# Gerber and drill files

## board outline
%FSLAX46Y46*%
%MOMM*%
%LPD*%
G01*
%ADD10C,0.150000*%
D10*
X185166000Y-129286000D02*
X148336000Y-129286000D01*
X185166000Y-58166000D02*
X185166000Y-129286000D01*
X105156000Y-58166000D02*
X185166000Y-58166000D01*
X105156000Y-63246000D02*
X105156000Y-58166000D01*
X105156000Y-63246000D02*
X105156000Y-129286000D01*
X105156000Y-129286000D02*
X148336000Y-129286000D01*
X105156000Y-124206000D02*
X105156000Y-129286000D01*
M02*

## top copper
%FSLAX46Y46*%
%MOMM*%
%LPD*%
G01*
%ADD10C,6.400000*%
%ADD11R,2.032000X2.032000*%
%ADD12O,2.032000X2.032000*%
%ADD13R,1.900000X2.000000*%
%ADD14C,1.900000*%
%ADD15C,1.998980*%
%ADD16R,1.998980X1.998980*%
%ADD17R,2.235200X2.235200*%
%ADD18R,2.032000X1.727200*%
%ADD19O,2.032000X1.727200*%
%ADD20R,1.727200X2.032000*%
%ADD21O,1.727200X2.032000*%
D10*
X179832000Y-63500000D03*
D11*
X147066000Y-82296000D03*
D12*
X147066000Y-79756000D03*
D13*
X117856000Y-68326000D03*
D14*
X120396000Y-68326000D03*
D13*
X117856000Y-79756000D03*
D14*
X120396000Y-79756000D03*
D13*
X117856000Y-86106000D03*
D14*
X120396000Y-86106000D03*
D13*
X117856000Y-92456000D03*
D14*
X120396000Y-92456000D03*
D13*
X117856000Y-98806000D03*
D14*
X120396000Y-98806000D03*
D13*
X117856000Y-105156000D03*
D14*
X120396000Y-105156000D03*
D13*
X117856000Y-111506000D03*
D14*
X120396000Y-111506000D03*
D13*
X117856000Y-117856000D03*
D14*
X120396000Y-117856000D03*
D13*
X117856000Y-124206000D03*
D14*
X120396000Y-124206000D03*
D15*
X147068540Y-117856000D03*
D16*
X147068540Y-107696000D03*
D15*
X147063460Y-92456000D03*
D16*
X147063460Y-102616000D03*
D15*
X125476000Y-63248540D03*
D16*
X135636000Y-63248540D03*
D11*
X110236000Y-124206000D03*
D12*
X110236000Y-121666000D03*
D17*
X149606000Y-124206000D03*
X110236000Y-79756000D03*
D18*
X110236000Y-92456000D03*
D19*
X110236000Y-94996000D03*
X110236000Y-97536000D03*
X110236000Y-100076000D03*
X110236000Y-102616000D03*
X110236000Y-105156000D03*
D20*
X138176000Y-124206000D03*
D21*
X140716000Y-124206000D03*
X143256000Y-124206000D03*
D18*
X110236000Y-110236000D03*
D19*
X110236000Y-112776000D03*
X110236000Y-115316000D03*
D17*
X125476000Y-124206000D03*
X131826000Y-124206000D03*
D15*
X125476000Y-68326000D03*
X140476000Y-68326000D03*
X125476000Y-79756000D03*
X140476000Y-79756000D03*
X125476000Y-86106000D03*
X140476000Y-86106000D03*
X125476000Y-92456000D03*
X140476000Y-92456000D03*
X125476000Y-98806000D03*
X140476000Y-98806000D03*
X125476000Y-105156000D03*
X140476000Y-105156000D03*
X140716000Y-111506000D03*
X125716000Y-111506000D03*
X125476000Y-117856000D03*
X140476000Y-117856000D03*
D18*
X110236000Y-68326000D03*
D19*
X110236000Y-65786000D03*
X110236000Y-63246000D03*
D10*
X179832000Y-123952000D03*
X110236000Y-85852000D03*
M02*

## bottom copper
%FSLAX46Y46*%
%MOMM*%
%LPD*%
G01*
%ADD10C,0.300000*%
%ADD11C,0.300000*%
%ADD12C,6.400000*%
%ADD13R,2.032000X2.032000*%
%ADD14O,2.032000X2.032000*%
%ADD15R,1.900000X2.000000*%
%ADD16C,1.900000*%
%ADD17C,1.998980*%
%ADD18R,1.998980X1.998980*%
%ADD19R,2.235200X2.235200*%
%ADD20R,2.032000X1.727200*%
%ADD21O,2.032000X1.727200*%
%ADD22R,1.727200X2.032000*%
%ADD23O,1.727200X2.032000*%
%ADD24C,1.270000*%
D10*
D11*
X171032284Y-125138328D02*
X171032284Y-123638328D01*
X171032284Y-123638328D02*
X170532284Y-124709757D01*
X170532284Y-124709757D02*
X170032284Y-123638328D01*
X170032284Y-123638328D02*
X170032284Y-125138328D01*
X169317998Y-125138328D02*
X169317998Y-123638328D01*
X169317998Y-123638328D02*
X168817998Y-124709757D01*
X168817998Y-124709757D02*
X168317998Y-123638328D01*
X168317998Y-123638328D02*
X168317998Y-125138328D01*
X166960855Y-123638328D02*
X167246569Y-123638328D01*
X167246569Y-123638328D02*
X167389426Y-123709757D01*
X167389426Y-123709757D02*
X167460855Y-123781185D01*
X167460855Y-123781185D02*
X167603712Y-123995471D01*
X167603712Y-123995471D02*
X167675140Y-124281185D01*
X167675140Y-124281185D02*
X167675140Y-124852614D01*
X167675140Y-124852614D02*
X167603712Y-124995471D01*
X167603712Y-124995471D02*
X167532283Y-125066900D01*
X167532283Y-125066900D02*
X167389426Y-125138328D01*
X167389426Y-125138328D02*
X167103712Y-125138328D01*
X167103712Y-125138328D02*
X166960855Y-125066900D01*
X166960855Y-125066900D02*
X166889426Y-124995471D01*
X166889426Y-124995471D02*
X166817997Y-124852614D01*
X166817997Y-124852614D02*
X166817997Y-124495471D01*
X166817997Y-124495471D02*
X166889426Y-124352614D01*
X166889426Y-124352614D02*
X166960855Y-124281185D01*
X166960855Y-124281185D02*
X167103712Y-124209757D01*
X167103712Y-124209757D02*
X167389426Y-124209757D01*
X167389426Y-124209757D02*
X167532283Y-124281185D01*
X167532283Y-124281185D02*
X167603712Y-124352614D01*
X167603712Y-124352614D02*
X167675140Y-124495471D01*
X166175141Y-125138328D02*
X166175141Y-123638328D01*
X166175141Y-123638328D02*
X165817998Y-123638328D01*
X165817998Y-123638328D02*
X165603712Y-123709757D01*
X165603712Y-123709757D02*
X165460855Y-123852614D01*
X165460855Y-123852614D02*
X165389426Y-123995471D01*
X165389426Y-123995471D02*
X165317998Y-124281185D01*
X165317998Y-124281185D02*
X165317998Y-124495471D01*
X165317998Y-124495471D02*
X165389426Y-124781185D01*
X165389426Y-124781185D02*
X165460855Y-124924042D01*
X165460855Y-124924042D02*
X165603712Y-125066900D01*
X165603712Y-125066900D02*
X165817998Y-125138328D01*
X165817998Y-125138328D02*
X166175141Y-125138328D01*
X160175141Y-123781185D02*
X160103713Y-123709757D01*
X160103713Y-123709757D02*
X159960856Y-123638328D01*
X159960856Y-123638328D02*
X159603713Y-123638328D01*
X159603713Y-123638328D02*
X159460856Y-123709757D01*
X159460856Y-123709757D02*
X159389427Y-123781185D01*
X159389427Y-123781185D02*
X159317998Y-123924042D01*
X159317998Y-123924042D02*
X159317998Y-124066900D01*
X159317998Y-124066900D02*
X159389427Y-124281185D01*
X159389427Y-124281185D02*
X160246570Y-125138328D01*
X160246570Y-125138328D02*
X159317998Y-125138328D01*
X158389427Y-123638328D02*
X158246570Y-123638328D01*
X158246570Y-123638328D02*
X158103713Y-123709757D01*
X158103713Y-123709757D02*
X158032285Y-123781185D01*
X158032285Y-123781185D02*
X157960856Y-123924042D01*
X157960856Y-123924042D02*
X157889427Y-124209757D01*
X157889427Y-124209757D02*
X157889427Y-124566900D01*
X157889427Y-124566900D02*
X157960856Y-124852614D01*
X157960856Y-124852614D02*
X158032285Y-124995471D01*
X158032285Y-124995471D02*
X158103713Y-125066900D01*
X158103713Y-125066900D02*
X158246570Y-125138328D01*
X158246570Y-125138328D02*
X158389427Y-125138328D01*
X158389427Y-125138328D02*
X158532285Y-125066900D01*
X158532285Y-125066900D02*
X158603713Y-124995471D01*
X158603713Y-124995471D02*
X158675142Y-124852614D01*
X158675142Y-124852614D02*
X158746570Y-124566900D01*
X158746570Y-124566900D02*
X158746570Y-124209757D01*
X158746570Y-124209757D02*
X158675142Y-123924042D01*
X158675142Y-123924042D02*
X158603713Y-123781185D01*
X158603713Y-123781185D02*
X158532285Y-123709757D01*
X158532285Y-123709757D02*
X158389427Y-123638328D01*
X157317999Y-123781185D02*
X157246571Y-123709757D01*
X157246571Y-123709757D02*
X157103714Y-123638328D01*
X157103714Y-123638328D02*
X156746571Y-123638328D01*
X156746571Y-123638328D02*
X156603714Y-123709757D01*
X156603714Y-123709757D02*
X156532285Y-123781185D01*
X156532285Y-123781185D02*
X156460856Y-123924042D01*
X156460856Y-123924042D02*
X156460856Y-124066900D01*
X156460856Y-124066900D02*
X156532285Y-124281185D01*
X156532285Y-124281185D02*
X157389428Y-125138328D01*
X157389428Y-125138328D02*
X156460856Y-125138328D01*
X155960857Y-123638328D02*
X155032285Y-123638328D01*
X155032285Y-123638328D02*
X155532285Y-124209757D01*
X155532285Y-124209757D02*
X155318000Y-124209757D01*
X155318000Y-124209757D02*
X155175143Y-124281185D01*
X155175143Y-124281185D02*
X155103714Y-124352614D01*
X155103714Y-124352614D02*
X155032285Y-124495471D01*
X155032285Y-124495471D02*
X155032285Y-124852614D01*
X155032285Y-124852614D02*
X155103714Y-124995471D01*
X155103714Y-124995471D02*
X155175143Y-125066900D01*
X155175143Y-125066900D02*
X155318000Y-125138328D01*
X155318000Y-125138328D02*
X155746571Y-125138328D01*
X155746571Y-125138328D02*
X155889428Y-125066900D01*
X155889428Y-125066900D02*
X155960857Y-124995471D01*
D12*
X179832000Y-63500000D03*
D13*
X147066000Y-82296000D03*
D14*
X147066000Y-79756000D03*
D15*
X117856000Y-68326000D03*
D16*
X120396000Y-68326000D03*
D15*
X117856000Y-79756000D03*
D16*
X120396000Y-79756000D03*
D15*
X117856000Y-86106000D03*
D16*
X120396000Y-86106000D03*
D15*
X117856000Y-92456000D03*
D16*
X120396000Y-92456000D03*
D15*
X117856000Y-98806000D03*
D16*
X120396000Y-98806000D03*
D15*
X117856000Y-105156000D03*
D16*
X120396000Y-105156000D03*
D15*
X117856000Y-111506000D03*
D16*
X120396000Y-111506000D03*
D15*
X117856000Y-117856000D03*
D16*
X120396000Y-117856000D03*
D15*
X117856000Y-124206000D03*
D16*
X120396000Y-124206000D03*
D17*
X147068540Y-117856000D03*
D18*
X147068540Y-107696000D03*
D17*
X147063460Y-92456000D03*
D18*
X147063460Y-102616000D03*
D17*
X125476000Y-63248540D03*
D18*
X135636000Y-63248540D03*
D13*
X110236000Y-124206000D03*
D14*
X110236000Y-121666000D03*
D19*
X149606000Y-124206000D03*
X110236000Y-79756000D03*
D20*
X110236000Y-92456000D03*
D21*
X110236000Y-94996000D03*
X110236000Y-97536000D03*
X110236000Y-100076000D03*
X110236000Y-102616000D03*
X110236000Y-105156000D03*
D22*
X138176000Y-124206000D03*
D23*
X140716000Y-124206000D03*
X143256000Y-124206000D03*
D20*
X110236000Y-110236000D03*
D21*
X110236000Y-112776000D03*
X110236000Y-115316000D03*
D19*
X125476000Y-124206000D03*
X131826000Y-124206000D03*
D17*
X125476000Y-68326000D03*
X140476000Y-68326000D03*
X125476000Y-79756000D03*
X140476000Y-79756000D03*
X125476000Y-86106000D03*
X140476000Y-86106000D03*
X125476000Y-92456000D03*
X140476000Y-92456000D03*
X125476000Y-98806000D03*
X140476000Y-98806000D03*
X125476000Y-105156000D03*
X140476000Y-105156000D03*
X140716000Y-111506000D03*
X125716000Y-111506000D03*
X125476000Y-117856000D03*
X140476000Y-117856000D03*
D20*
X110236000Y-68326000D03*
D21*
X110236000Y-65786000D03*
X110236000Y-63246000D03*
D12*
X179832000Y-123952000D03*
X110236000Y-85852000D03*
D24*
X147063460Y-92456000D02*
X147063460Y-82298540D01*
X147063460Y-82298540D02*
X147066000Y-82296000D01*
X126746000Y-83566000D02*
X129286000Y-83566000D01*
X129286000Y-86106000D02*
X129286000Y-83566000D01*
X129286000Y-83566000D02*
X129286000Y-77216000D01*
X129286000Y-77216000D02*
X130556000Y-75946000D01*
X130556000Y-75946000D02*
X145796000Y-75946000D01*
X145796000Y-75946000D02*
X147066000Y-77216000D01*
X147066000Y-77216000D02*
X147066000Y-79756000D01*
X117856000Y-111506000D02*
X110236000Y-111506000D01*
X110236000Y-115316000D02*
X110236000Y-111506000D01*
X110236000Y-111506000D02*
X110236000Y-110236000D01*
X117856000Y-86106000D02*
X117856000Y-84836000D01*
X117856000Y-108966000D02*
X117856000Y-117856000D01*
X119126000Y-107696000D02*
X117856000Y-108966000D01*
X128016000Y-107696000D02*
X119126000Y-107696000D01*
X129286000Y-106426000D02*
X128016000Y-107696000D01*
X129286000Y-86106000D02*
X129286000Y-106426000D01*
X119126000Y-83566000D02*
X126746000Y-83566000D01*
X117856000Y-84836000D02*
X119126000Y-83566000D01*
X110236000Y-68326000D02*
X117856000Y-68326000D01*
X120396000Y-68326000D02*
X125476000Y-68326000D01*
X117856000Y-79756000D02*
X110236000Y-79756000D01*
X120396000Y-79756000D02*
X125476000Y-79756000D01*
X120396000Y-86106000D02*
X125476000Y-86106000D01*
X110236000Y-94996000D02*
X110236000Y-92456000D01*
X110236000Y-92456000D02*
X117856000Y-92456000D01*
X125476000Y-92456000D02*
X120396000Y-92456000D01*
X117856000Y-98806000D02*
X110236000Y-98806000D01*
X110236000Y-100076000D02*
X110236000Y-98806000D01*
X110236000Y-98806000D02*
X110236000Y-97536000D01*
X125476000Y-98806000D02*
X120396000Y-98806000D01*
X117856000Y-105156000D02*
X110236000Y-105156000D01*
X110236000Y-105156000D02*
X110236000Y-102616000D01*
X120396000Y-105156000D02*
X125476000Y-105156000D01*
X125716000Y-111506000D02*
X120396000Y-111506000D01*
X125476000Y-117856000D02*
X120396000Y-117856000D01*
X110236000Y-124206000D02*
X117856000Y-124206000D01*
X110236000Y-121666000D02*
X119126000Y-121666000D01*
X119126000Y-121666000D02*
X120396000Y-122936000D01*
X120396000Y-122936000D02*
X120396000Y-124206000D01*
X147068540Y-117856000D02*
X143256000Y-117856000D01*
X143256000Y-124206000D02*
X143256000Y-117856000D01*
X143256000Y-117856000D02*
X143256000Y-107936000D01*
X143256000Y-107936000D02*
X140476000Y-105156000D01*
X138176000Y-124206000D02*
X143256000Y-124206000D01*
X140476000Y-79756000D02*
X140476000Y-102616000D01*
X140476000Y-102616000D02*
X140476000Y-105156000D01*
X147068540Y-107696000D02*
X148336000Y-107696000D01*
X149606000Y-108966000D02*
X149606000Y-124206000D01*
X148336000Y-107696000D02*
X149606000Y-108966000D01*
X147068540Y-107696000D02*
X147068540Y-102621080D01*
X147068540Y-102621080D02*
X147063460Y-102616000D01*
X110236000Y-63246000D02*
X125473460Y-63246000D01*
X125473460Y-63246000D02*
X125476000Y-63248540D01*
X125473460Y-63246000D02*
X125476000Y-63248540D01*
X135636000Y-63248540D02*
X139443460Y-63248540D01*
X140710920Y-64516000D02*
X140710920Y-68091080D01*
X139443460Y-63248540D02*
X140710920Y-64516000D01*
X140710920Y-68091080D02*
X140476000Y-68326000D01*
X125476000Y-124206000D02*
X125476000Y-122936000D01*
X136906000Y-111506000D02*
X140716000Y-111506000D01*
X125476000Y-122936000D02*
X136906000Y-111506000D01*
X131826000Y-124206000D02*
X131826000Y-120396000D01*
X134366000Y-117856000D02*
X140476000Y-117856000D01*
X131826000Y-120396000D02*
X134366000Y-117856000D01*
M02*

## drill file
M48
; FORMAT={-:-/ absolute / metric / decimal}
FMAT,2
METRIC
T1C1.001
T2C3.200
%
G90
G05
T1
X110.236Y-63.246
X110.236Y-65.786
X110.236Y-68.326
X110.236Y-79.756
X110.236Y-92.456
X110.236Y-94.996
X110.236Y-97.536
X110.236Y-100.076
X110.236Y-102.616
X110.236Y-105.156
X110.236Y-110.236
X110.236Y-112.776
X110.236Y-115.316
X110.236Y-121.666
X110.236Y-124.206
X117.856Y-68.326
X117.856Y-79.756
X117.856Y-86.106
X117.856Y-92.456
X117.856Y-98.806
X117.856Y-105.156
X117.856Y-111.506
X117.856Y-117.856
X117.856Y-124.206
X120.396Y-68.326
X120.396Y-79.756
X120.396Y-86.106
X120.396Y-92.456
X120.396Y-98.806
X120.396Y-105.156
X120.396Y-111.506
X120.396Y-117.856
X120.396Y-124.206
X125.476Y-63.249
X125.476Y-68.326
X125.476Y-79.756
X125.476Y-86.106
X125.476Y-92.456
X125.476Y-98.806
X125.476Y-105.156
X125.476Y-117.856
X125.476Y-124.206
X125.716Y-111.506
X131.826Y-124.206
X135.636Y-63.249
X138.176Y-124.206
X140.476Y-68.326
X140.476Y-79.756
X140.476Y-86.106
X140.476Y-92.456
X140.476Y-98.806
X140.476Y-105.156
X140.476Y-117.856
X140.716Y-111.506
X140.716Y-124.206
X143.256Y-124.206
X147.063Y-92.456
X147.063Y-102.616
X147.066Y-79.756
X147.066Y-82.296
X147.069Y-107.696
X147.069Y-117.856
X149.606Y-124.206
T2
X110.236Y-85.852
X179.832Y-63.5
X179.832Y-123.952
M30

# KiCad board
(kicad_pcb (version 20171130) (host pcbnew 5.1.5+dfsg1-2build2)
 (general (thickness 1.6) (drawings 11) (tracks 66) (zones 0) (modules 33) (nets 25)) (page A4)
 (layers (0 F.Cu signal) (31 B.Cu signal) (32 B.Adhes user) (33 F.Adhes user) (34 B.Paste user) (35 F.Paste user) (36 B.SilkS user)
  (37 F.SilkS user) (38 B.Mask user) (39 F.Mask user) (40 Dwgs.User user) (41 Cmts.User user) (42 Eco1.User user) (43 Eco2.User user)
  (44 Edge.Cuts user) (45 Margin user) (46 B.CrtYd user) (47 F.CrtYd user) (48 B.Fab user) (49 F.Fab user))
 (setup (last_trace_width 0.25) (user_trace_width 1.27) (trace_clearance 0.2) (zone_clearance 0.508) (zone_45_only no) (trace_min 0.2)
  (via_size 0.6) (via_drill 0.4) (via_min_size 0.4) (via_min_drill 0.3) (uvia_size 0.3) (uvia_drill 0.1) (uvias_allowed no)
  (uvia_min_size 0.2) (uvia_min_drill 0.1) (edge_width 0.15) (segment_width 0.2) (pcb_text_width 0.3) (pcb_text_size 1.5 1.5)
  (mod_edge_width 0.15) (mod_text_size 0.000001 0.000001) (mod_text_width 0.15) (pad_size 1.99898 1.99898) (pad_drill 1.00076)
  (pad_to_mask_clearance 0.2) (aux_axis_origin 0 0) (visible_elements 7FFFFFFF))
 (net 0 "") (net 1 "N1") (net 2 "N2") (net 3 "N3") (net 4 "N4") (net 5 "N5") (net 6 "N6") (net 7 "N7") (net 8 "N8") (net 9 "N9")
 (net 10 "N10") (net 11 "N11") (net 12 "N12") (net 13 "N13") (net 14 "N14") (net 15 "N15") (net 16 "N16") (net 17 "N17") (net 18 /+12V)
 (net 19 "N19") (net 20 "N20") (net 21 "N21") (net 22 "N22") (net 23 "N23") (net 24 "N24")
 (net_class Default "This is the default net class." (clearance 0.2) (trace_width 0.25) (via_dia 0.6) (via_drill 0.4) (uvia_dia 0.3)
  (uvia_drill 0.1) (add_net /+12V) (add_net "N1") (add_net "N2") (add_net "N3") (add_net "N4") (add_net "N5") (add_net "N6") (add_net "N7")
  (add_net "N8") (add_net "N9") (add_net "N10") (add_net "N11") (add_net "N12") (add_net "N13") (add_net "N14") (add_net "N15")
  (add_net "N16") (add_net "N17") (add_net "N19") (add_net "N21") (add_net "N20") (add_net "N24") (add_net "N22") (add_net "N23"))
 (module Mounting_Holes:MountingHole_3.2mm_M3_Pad (layer F.Cu) (at 179.832 63.5)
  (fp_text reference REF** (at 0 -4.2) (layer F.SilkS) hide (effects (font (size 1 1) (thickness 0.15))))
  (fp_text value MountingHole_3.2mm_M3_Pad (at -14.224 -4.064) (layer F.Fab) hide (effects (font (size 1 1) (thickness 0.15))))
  (pad 1 thru_hole circle (at 0 0) (size 6.4 6.4) (drill 3.2) (layers *.Cu *.Mask)))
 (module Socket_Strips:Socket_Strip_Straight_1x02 (layer F.Cu) (at 147.066 82.296 90)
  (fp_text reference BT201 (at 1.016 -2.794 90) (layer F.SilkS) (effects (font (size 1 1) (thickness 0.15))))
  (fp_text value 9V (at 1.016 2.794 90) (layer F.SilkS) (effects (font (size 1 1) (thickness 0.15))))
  (pad 1 thru_hole rect (at 0 0 90) (size 2.032 2.032) (drill 1.00076) (layers *.Cu *.Mask) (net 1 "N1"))
  (pad 2 thru_hole oval (at 2.54 0 90) (size 2.032 2.032) (drill 1.00076) (layers *.Cu *.Mask) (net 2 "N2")))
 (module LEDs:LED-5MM (layer F.Cu) (at 117.856 68.326)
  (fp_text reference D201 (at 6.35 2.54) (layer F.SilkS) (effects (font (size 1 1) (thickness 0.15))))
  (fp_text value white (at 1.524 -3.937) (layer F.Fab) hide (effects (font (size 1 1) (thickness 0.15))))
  (pad 1 thru_hole rect (at 0 0 90) (size 2 1.9) (drill 1.00076) (layers *.Cu *.Mask) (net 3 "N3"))
  (pad 2 thru_hole circle (at 2.54 0) (size 1.9 1.9) (drill 1.00076) (layers *.Cu *.Mask) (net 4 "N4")))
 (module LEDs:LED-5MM (layer F.Cu) (at 117.856 79.756)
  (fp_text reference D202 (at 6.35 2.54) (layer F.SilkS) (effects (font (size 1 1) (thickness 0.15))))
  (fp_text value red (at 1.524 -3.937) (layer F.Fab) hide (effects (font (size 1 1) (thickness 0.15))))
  (pad 1 thru_hole rect (at 0 0 90) (size 2 1.9) (drill 1.00076) (layers *.Cu *.Mask) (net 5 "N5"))
  (pad 2 thru_hole circle (at 2.54 0) (size 1.9 1.9) (drill 1.00076) (layers *.Cu *.Mask) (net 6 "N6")))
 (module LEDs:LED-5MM (layer F.Cu) (at 117.856 86.106)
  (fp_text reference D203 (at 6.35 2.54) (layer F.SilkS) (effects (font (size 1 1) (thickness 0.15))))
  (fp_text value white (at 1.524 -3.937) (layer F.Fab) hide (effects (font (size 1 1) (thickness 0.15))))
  (pad 1 thru_hole rect (at 0 0 90) (size 2 1.9) (drill 1.00076) (layers *.Cu *.Mask) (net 2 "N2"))
  (pad 2 thru_hole circle (at 2.54 0) (size 1.9 1.9) (drill 1.00076) (layers *.Cu *.Mask) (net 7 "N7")))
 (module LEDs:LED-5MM (layer F.Cu) (at 117.856 92.456)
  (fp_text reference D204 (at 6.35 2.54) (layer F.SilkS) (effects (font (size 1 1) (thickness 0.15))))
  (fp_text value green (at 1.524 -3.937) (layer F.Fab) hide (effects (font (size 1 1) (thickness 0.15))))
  (pad 1 thru_hole rect (at 0 0 90) (size 2 1.9) (drill 1.00076) (layers *.Cu *.Mask) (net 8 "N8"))
  (pad 2 thru_hole circle (at 2.54 0) (size 1.9 1.9) (drill 1.00076) (layers *.Cu *.Mask) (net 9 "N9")))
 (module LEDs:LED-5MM (layer F.Cu) (at 117.856 98.806)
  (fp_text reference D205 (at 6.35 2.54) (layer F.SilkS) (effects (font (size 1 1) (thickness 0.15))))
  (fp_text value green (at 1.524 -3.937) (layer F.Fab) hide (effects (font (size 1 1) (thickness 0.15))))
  (pad 1 thru_hole rect (at 0 0 90) (size 2 1.9) (drill 1.00076) (layers *.Cu *.Mask) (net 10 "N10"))
  (pad 2 thru_hole circle (at 2.54 0) (size 1.9 1.9) (drill 1.00076) (layers *.Cu *.Mask) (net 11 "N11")))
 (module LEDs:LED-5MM (layer F.Cu) (at 117.856 105.156)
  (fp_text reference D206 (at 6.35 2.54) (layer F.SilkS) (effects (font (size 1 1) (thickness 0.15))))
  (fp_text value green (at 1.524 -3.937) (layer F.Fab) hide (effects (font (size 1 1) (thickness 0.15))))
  (pad 1 thru_hole rect (at 0 0 90) (size 2 1.9) (drill 1.00076) (layers *.Cu *.Mask) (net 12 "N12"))
  (pad 2 thru_hole circle (at 2.54 0) (size 1.9 1.9) (drill 1.00076) (layers *.Cu *.Mask) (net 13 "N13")))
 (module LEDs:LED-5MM (layer F.Cu) (at 117.856 111.506)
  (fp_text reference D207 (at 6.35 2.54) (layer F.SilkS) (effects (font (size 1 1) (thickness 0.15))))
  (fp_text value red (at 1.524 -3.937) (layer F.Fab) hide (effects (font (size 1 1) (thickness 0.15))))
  (pad 1 thru_hole rect (at 0 0 90) (size 2 1.9) (drill 1.00076) (layers *.Cu *.Mask) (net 2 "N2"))
  (pad 2 thru_hole circle (at 2.54 0) (size 1.9 1.9) (drill 1.00076) (layers *.Cu *.Mask) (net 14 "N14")))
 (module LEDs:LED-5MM (layer F.Cu) (at 117.856 117.856)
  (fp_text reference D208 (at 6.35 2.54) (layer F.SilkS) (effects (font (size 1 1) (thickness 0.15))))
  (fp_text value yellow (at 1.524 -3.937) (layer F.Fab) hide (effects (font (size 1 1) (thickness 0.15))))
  (pad 1 thru_hole rect (at 0 0 90) (size 2 1.9) (drill 1.00076) (layers *.Cu *.Mask) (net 2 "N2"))
  (pad 2 thru_hole circle (at 2.54 0) (size 1.9 1.9) (drill 1.00076) (layers *.Cu *.Mask) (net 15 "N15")))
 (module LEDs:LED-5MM (layer F.Cu) (at 117.856 124.206)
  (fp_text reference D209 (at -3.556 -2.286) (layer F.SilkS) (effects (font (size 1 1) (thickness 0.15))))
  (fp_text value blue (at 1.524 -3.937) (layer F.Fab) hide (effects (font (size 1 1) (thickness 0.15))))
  (pad 1 thru_hole rect (at 0 0 90) (size 2 1.9) (drill 1.00076) (layers *.Cu *.Mask) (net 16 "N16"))
  (pad 2 thru_hole circle (at 2.54 0) (size 1.9 1.9) (drill 1.00076) (layers *.Cu *.Mask) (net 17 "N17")))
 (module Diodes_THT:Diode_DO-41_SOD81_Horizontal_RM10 (layer F.Cu) (at 147.066 107.696 270)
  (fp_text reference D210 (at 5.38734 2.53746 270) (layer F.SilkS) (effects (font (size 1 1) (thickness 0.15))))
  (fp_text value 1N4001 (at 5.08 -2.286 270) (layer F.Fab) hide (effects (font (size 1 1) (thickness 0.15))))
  (pad 2 thru_hole circle (at 10.16 -0.00254 90) (size 1.99898 1.99898) (drill 1.00076) (layers *.Cu *.Mask) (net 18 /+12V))
  (pad 1 thru_hole rect (at 0 -0.00254 90) (size 1.99898 1.99898) (drill 1.00076) (layers *.Cu *.Mask) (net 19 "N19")))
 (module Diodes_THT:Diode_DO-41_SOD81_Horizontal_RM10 (layer F.Cu) (at 147.066 102.616 90)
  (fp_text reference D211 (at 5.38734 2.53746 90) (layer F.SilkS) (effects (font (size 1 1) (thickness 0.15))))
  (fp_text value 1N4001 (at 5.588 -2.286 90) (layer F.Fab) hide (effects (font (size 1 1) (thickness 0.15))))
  (pad 2 thru_hole circle (at 10.16 -0.00254 270) (size 1.99898 1.99898) (drill 1.00076) (layers *.Cu *.Mask) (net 1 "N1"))
  (pad 1 thru_hole rect (at 0 -0.00254 270) (size 1.99898 1.99898) (drill 1.00076) (layers *.Cu *.Mask) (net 19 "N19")))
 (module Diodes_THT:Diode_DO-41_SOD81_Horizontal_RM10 (layer F.Cu) (at 135.636 63.246 180)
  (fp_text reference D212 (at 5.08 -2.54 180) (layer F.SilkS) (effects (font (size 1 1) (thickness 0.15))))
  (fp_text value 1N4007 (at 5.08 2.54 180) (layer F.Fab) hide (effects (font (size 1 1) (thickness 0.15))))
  (pad 2 thru_hole circle (at 10.16 -0.00254) (size 1.99898 1.99898) (drill 1.00076) (layers *.Cu *.Mask) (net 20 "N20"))
  (pad 1 thru_hole rect (at 0 -0.00254) (size 1.99898 1.99898) (drill 1.00076) (layers *.Cu *.Mask) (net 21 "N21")))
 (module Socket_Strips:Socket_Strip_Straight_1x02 (layer F.Cu) (at 110.236 124.206 90)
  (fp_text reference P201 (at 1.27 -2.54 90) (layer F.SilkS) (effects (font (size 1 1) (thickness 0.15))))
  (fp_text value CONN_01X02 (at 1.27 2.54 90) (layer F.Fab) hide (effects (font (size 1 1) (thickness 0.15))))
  (pad 1 thru_hole rect (at 0 0 90) (size 2.032 2.032) (drill 1.00076) (layers *.Cu *.Mask) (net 16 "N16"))
  (pad 2 thru_hole oval (at 2.54 0 90) (size 2.032 2.032) (drill 1.00076) (layers *.Cu *.Mask) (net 17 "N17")))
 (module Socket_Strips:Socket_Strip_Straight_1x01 (layer F.Cu) (at 149.606 124.206)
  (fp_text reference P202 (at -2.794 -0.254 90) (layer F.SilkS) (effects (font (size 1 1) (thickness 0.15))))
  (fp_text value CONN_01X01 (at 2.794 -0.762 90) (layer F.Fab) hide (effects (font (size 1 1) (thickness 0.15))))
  (pad 1 thru_hole rect (at 0 0) (size 2.2352 2.2352) (drill 1.00076) (layers *.Cu *.Mask) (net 19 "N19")))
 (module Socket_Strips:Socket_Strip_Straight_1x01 (layer F.Cu) (at 110.236 79.756 270)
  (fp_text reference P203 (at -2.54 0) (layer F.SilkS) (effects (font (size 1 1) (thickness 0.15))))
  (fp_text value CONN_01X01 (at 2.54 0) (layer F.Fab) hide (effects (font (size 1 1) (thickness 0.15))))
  (pad 1 thru_hole rect (at 0 0 270) (size 2.2352 2.2352) (drill 1.00076) (layers *.Cu *.Mask) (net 5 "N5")))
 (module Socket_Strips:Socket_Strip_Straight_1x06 (layer F.Cu) (at 110.236 92.456 270)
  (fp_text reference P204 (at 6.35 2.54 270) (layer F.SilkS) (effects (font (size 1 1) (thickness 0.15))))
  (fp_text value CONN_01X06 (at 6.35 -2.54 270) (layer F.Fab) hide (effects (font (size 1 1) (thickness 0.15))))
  (pad 1 thru_hole rect (at 0 0 270) (size 1.7272 2.032) (drill 1.00076) (layers *.Cu *.Mask) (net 8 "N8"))
  (pad 2 thru_hole oval (at 2.54 0 270) (size 1.7272 2.032) (drill 1.00076) (layers *.Cu *.Mask) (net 8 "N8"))
  (pad 3 thru_hole oval (at 5.08 0 270) (size 1.7272 2.032) (drill 1.00076) (layers *.Cu *.Mask) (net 10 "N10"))
  (pad 4 thru_hole oval (at 7.62 0 270) (size 1.7272 2.032) (drill 1.00076) (layers *.Cu *.Mask) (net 10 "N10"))
  (pad 5 thru_hole oval (at 10.16 0 270) (size 1.7272 2.032) (drill 1.00076) (layers *.Cu *.Mask) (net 12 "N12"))
  (pad 6 thru_hole oval (at 12.7 0 270) (size 1.7272 2.032) (drill 1.00076) (layers *.Cu *.Mask) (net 12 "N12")))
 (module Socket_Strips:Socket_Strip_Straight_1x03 (layer F.Cu) (at 138.176 124.206)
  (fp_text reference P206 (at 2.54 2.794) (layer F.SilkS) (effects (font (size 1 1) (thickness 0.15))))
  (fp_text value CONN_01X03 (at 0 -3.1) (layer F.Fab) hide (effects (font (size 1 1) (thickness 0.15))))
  (pad 1 thru_hole rect (at 0 0) (size 1.7272 2.032) (drill 1.00076) (layers *.Cu *.Mask) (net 18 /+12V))
  (pad 2 thru_hole oval (at 2.54 0) (size 1.7272 2.032) (drill 1.00076) (layers *.Cu *.Mask) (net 18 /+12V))
  (pad 3 thru_hole oval (at 5.08 0) (size 1.7272 2.032) (drill 1.00076) (layers *.Cu *.Mask) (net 18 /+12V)))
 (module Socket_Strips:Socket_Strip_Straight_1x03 (layer F.Cu) (at 110.236 110.236 270)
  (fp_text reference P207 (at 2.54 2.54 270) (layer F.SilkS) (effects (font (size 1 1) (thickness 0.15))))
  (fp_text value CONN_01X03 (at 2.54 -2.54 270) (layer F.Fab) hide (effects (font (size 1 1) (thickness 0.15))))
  (pad 1 thru_hole rect (at 0 0 270) (size 1.7272 2.032) (drill 1.00076) (layers *.Cu *.Mask) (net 2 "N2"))
  (pad 2 thru_hole oval (at 2.54 0 270) (size 1.7272 2.032) (drill 1.00076) (layers *.Cu *.Mask) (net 2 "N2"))
  (pad 3 thru_hole oval (at 5.08 0 270) (size 1.7272 2.032) (drill 1.00076) (layers *.Cu *.Mask) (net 2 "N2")))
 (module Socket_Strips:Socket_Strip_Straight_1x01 (layer F.Cu) (at 125.476 124.206)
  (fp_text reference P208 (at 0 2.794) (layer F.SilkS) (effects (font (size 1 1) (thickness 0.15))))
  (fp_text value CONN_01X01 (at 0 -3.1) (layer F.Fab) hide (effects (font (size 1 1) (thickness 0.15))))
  (pad 1 thru_hole rect (at 0 0) (size 2.2352 2.2352) (drill 1.00076) (layers *.Cu *.Mask) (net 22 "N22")))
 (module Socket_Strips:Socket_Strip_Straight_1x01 (layer F.Cu) (at 131.826 124.206)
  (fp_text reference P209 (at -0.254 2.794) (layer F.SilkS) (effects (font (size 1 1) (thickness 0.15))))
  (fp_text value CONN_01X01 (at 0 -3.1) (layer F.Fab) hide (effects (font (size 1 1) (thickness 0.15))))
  (pad 1 thru_hole rect (at 0 0) (size 2.2352 2.2352) (drill 1.00076) (layers *.Cu *.Mask) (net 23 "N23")))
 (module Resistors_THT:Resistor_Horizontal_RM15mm (layer F.Cu) (at 125.476 68.326)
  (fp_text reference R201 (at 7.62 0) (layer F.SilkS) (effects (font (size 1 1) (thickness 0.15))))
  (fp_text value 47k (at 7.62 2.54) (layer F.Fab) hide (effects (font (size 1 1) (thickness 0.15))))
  (pad 1 thru_hole circle (at 0 0) (size 1.99898 1.99898) (drill 1.00076) (layers *.Cu *.SilkS *.Mask) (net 4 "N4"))
  (pad 2 thru_hole circle (at 15 0) (size 1.99898 1.99898) (drill 1.00076) (layers *.Cu *.SilkS *.Mask) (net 21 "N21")))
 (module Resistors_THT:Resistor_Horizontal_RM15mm (layer F.Cu) (at 125.476 79.756)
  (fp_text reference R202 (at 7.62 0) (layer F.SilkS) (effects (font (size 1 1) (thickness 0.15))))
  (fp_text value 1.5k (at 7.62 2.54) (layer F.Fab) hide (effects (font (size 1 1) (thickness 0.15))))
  (pad 1 thru_hole circle (at 0 0) (size 1.99898 1.99898) (drill 1.00076) (layers *.Cu *.SilkS *.Mask) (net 6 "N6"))
  (pad 2 thru_hole circle (at 15 0) (size 1.99898 1.99898) (drill 1.00076) (layers *.Cu *.SilkS *.Mask) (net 18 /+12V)))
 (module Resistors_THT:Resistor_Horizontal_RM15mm (layer F.Cu) (at 125.476 86.106)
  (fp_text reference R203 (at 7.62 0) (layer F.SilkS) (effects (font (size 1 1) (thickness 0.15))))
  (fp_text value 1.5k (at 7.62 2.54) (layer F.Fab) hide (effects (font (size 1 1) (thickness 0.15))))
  (pad 1 thru_hole circle (at 0 0) (size 1.99898 1.99898) (drill 1.00076) (layers *.Cu *.SilkS *.Mask) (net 7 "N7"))
  (pad 2 thru_hole circle (at 15 0) (size 1.99898 1.99898) (drill 1.00076) (layers *.Cu *.SilkS *.Mask) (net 18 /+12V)))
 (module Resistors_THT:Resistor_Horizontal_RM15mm (layer F.Cu) (at 125.476 92.456)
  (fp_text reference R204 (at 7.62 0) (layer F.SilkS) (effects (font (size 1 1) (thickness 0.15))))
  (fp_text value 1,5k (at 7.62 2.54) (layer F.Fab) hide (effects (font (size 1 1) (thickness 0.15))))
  (pad 1 thru_hole circle (at 0 0) (size 1.99898 1.99898) (drill 1.00076) (layers *.Cu *.SilkS *.Mask) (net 9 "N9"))
  (pad 2 thru_hole circle (at 15 0) (size 1.99898 1.99898) (drill 1.00076) (layers *.Cu *.SilkS *.Mask) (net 18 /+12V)))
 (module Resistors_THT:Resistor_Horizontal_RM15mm (layer F.Cu) (at 125.476 98.806)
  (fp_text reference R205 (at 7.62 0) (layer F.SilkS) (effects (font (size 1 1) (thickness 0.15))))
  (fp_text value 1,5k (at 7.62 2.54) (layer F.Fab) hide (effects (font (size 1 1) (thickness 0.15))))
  (pad 1 thru_hole circle (at 0 0) (size 1.99898 1.99898) (drill 1.00076) (layers *.Cu *.SilkS *.Mask) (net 11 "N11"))
  (pad 2 thru_hole circle (at 15 0) (size 1.99898 1.99898) (drill 1.00076) (layers *.Cu *.SilkS *.Mask) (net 18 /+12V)))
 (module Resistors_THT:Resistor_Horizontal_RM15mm (layer F.Cu) (at 125.476 105.156)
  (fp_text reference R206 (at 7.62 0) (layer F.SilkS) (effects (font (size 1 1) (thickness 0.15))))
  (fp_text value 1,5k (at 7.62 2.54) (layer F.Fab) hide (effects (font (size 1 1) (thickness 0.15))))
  (pad 1 thru_hole circle (at 0 0) (size 1.99898 1.99898) (drill 1.00076) (layers *.Cu *.SilkS *.Mask) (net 13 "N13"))
  (pad 2 thru_hole circle (at 15 0) (size 1.99898 1.99898) (drill 1.00076) (layers *.Cu *.SilkS *.Mask) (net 18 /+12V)))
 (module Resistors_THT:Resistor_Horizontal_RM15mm (layer F.Cu) (at 140.716 111.506 180)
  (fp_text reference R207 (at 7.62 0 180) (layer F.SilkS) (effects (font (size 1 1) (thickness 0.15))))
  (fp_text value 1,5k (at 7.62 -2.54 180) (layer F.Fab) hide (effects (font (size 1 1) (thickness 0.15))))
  (pad 1 thru_hole circle (at 0 0 180) (size 1.99898 1.99898) (drill 1.00076) (layers *.Cu *.SilkS *.Mask) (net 22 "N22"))
  (pad 2 thru_hole circle (at 15 0 180) (size 1.99898 1.99898) (drill 1.00076) (layers *.Cu *.SilkS *.Mask) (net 14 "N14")))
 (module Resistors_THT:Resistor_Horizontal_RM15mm (layer F.Cu) (at 125.476 117.856)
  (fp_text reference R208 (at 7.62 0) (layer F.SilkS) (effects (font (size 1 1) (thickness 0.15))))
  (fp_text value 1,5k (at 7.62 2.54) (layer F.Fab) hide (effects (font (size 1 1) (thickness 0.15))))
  (pad 1 thru_hole circle (at 0 0) (size 1.99898 1.99898) (drill 1.00076) (layers *.Cu *.SilkS *.Mask) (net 15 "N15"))
  (pad 2 thru_hole circle (at 15 0) (size 1.99898 1.99898) (drill 1.00076) (layers *.Cu *.SilkS *.Mask) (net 23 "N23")))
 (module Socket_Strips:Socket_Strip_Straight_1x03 (layer F.Cu) (at 110.236 68.326 90)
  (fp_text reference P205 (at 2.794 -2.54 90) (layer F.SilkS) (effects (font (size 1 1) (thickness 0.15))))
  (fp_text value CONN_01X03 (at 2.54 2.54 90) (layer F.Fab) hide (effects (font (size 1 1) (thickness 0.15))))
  (pad 1 thru_hole rect (at 0 0 90) (size 1.7272 2.032) (drill 1.00076) (layers *.Cu *.Mask) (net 3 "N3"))
  (pad 2 thru_hole oval (at 2.54 0 90) (size 1.7272 2.032) (drill 1.00076) (layers *.Cu *.Mask) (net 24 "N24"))
  (pad 3 thru_hole oval (at 5.08 0 90) (size 1.7272 2.032) (drill 1.00076) (layers *.Cu *.Mask) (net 20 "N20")))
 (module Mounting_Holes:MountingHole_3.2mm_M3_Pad (layer F.Cu) (at 179.832 123.952)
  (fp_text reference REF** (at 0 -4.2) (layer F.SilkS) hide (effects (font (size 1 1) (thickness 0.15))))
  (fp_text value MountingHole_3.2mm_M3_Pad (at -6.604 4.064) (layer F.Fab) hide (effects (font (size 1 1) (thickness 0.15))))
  (pad 1 thru_hole circle (at 0 0) (size 6.4 6.4) (drill 3.2) (layers *.Cu *.Mask)))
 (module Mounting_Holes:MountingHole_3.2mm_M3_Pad (layer F.Cu) (at 110.236 85.852)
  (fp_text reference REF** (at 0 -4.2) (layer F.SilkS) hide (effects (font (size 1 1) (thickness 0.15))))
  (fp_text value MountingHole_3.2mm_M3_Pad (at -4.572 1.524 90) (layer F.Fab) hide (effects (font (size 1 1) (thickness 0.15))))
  (pad 1 thru_hole circle (at 0 0) (size 6.4 6.4) (drill 3.2) (layers *.Cu *.Mask)))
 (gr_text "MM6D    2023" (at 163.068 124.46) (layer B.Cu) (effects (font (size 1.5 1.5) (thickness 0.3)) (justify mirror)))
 (gr_line (start 185.166 129.286) (end 148.336 129.286) (angle 90) (layer Edge.Cuts) (width 0.15))
 (gr_line (start 185.166 58.166) (end 185.166 129.286) (angle 90) (layer Edge.Cuts) (width 0.15))
 (gr_line (start 105.156 58.166) (end 185.166 58.166) (angle 90) (layer Edge.Cuts) (width 0.15))
 (gr_line (start 105.156 63.246) (end 105.156 58.166) (angle 90) (layer Edge.Cuts) (width 0.15))
 (gr_line (start 105.156 63.246) (end 105.156 129.286) (angle 90) (layer Edge.Cuts) (width 0.15))
 (gr_line (start 105.156 129.286) (end 148.336 129.286) (angle 90) (layer Edge.Cuts) (width 0.15))
 (gr_line (start 105.156 124.206) (end 105.156 129.286) (angle 90) (layer Edge.Cuts) (width 0.15))
 (segment (start 147.06346 92.456) (end 147.06346 82.29854) (width 1.27) (layer B.Cu) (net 1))
 (segment (start 147.06346 82.29854) (end 147.066 82.296) (width 1.27) (layer B.Cu) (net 1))
 (segment (start 126.746 83.566) (end 129.286 83.566) (width 1.27) (layer B.Cu) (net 2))
 (segment (start 129.286 86.106) (end 129.286 83.566) (width 1.27) (layer B.Cu) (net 2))
 (segment (start 129.286 83.566) (end 129.286 77.216) (width 1.27) (layer B.Cu) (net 2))
 (segment (start 129.286 77.216) (end 130.556 75.946) (width 1.27) (layer B.Cu) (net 2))
 (segment (start 130.556 75.946) (end 145.796 75.946) (width 1.27) (layer B.Cu) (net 2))
 (segment (start 145.796 75.946) (end 147.066 77.216) (width 1.27) (layer B.Cu) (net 2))
 (segment (start 147.066 77.216) (end 147.066 79.756) (width 1.27) (layer B.Cu) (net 2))
 (segment (start 117.856 111.506) (end 110.236 111.506) (width 1.27) (layer B.Cu) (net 2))
 (segment (start 110.236 115.316) (end 110.236 111.506) (width 1.27) (layer B.Cu) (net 2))
 (segment (start 110.236 111.506) (end 110.236 110.236) (width 1.27) (layer B.Cu) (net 2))
 (segment (start 117.856 86.106) (end 117.856 84.836) (width 1.27) (layer B.Cu) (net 2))
 (segment (start 117.856 108.966) (end 117.856 117.856) (width 1.27) (layer B.Cu) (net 2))
 (segment (start 119.126 107.696) (end 117.856 108.966) (width 1.27) (layer B.Cu) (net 2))
 (segment (start 128.016 107.696) (end 119.126 107.696) (width 1.27) (layer B.Cu) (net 2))
 (segment (start 129.286 106.426) (end 128.016 107.696) (width 1.27) (layer B.Cu) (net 2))
 (segment (start 129.286 86.106) (end 129.286 106.426) (width 1.27) (layer B.Cu) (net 2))
 (segment (start 119.126 83.566) (end 126.746 83.566) (width 1.27) (layer B.Cu) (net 2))
 (segment (start 117.856 84.836) (end 119.126 83.566) (width 1.27) (layer B.Cu) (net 2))
 (segment (start 110.236 68.326) (end 117.856 68.326) (width 1.27) (layer B.Cu) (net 3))
 (segment (start 120.396 68.326) (end 125.476 68.326) (width 1.27) (layer B.Cu) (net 4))
 (segment (start 117.856 79.756) (end 110.236 79.756) (width 1.27) (layer B.Cu) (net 5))
 (segment (start 120.396 79.756) (end 125.476 79.756) (width 1.27) (layer B.Cu) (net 6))
 (segment (start 120.396 86.106) (end 125.476 86.106) (width 1.27) (layer B.Cu) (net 7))
 (segment (start 110.236 94.996) (end 110.236 92.456) (width 1.27) (layer B.Cu) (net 8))
 (segment (start 110.236 92.456) (end 117.856 92.456) (width 1.27) (layer B.Cu) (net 8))
 (segment (start 125.476 92.456) (end 120.396 92.456) (width 1.27) (layer B.Cu) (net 9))
 (segment (start 117.856 98.806) (end 110.236 98.806) (width 1.27) (layer B.Cu) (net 10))
 (segment (start 110.236 100.076) (end 110.236 98.806) (width 1.27) (layer B.Cu) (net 10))
 (segment (start 110.236 98.806) (end 110.236 97.536) (width 1.27) (layer B.Cu) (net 10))
 (segment (start 125.476 98.806) (end 120.396 98.806) (width 1.27) (layer B.Cu) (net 11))
 (segment (start 117.856 105.156) (end 110.236 105.156) (width 1.27) (layer B.Cu) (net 12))
 (segment (start 110.236 105.156) (end 110.236 102.616) (width 1.27) (layer B.Cu) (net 12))
 (segment (start 120.396 105.156) (end 125.476 105.156) (width 1.27) (layer B.Cu) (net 13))
 (segment (start 125.716 111.506) (end 120.396 111.506) (width 1.27) (layer B.Cu) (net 14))
 (segment (start 125.476 117.856) (end 120.396 117.856) (width 1.27) (layer B.Cu) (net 15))
 (segment (start 110.236 124.206) (end 117.856 124.206) (width 1.27) (layer B.Cu) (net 16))
 (segment (start 110.236 121.666) (end 119.126 121.666) (width 1.27) (layer B.Cu) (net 17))
 (segment (start 119.126 121.666) (end 120.396 122.936) (width 1.27) (layer B.Cu) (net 17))
 (segment (start 120.396 122.936) (end 120.396 124.206) (width 1.27) (layer B.Cu) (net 17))
 (segment (start 147.06854 117.856) (end 143.256 117.856) (width 1.27) (layer B.Cu) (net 18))
 (segment (start 143.256 124.206) (end 143.256 117.856) (width 1.27) (layer B.Cu) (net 18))
 (segment (start 143.256 117.856) (end 143.256 107.936) (width 1.27) (layer B.Cu) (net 18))
 (segment (start 143.256 107.936) (end 140.476 105.156) (width 1.27) (layer B.Cu) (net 18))
 (segment (start 138.176 124.206) (end 143.256 124.206) (width 1.27) (layer B.Cu) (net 18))
 (segment (start 140.476 79.756) (end 140.476 102.616) (width 1.27) (layer B.Cu) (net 18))
 (segment (start 140.476 102.616) (end 140.476 105.156) (width 1.27) (layer B.Cu) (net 18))
 (segment (start 147.06854 107.696) (end 148.336 107.696) (width 1.27) (layer B.Cu) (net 19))
 (segment (start 149.606 108.966) (end 149.606 124.206) (width 1.27) (layer B.Cu) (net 19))
 (segment (start 148.336 107.696) (end 149.606 108.966) (width 1.27) (layer B.Cu) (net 19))
 (segment (start 147.06854 107.696) (end 147.06854 102.62108) (width 1.27) (layer B.Cu) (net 19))
 (segment (start 147.06854 102.62108) (end 147.06346 102.616) (width 1.27) (layer B.Cu) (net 19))
 (segment (start 110.236 63.246) (end 125.47346 63.246) (width 1.27) (layer B.Cu) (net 20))
 (segment (start 125.47346 63.246) (end 125.476 63.24854) (width 1.27) (layer B.Cu) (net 20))
 (segment (start 125.47346 63.246) (end 125.476 63.24854) (width 1.27) (layer B.Cu) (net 20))
 (segment (start 135.636 63.24854) (end 139.44346 63.24854) (width 1.27) (layer B.Cu) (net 21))
 (segment (start 140.71092 64.516) (end 140.71092 68.09108) (width 1.27) (layer B.Cu) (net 21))
 (segment (start 139.44346 63.24854) (end 140.71092 64.516) (width 1.27) (layer B.Cu) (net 21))
 (segment (start 140.71092 68.09108) (end 140.476 68.326) (width 1.27) (layer B.Cu) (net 21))
 (segment (start 125.476 124.206) (end 125.476 122.936) (width 1.27) (layer B.Cu) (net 22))
 (segment (start 136.906 111.506) (end 140.716 111.506) (width 1.27) (layer B.Cu) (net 22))
 (segment (start 125.476 122.936) (end 136.906 111.506) (width 1.27) (layer B.Cu) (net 22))
 (segment (start 131.826 124.206) (end 131.826 120.396) (width 1.27) (layer B.Cu) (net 23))
 (segment (start 134.366 117.856) (end 140.476 117.856) (width 1.27) (layer B.Cu) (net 23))
 (segment (start 131.826 120.396) (end 134.366 117.856) (width 1.27) (layer B.Cu) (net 23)))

